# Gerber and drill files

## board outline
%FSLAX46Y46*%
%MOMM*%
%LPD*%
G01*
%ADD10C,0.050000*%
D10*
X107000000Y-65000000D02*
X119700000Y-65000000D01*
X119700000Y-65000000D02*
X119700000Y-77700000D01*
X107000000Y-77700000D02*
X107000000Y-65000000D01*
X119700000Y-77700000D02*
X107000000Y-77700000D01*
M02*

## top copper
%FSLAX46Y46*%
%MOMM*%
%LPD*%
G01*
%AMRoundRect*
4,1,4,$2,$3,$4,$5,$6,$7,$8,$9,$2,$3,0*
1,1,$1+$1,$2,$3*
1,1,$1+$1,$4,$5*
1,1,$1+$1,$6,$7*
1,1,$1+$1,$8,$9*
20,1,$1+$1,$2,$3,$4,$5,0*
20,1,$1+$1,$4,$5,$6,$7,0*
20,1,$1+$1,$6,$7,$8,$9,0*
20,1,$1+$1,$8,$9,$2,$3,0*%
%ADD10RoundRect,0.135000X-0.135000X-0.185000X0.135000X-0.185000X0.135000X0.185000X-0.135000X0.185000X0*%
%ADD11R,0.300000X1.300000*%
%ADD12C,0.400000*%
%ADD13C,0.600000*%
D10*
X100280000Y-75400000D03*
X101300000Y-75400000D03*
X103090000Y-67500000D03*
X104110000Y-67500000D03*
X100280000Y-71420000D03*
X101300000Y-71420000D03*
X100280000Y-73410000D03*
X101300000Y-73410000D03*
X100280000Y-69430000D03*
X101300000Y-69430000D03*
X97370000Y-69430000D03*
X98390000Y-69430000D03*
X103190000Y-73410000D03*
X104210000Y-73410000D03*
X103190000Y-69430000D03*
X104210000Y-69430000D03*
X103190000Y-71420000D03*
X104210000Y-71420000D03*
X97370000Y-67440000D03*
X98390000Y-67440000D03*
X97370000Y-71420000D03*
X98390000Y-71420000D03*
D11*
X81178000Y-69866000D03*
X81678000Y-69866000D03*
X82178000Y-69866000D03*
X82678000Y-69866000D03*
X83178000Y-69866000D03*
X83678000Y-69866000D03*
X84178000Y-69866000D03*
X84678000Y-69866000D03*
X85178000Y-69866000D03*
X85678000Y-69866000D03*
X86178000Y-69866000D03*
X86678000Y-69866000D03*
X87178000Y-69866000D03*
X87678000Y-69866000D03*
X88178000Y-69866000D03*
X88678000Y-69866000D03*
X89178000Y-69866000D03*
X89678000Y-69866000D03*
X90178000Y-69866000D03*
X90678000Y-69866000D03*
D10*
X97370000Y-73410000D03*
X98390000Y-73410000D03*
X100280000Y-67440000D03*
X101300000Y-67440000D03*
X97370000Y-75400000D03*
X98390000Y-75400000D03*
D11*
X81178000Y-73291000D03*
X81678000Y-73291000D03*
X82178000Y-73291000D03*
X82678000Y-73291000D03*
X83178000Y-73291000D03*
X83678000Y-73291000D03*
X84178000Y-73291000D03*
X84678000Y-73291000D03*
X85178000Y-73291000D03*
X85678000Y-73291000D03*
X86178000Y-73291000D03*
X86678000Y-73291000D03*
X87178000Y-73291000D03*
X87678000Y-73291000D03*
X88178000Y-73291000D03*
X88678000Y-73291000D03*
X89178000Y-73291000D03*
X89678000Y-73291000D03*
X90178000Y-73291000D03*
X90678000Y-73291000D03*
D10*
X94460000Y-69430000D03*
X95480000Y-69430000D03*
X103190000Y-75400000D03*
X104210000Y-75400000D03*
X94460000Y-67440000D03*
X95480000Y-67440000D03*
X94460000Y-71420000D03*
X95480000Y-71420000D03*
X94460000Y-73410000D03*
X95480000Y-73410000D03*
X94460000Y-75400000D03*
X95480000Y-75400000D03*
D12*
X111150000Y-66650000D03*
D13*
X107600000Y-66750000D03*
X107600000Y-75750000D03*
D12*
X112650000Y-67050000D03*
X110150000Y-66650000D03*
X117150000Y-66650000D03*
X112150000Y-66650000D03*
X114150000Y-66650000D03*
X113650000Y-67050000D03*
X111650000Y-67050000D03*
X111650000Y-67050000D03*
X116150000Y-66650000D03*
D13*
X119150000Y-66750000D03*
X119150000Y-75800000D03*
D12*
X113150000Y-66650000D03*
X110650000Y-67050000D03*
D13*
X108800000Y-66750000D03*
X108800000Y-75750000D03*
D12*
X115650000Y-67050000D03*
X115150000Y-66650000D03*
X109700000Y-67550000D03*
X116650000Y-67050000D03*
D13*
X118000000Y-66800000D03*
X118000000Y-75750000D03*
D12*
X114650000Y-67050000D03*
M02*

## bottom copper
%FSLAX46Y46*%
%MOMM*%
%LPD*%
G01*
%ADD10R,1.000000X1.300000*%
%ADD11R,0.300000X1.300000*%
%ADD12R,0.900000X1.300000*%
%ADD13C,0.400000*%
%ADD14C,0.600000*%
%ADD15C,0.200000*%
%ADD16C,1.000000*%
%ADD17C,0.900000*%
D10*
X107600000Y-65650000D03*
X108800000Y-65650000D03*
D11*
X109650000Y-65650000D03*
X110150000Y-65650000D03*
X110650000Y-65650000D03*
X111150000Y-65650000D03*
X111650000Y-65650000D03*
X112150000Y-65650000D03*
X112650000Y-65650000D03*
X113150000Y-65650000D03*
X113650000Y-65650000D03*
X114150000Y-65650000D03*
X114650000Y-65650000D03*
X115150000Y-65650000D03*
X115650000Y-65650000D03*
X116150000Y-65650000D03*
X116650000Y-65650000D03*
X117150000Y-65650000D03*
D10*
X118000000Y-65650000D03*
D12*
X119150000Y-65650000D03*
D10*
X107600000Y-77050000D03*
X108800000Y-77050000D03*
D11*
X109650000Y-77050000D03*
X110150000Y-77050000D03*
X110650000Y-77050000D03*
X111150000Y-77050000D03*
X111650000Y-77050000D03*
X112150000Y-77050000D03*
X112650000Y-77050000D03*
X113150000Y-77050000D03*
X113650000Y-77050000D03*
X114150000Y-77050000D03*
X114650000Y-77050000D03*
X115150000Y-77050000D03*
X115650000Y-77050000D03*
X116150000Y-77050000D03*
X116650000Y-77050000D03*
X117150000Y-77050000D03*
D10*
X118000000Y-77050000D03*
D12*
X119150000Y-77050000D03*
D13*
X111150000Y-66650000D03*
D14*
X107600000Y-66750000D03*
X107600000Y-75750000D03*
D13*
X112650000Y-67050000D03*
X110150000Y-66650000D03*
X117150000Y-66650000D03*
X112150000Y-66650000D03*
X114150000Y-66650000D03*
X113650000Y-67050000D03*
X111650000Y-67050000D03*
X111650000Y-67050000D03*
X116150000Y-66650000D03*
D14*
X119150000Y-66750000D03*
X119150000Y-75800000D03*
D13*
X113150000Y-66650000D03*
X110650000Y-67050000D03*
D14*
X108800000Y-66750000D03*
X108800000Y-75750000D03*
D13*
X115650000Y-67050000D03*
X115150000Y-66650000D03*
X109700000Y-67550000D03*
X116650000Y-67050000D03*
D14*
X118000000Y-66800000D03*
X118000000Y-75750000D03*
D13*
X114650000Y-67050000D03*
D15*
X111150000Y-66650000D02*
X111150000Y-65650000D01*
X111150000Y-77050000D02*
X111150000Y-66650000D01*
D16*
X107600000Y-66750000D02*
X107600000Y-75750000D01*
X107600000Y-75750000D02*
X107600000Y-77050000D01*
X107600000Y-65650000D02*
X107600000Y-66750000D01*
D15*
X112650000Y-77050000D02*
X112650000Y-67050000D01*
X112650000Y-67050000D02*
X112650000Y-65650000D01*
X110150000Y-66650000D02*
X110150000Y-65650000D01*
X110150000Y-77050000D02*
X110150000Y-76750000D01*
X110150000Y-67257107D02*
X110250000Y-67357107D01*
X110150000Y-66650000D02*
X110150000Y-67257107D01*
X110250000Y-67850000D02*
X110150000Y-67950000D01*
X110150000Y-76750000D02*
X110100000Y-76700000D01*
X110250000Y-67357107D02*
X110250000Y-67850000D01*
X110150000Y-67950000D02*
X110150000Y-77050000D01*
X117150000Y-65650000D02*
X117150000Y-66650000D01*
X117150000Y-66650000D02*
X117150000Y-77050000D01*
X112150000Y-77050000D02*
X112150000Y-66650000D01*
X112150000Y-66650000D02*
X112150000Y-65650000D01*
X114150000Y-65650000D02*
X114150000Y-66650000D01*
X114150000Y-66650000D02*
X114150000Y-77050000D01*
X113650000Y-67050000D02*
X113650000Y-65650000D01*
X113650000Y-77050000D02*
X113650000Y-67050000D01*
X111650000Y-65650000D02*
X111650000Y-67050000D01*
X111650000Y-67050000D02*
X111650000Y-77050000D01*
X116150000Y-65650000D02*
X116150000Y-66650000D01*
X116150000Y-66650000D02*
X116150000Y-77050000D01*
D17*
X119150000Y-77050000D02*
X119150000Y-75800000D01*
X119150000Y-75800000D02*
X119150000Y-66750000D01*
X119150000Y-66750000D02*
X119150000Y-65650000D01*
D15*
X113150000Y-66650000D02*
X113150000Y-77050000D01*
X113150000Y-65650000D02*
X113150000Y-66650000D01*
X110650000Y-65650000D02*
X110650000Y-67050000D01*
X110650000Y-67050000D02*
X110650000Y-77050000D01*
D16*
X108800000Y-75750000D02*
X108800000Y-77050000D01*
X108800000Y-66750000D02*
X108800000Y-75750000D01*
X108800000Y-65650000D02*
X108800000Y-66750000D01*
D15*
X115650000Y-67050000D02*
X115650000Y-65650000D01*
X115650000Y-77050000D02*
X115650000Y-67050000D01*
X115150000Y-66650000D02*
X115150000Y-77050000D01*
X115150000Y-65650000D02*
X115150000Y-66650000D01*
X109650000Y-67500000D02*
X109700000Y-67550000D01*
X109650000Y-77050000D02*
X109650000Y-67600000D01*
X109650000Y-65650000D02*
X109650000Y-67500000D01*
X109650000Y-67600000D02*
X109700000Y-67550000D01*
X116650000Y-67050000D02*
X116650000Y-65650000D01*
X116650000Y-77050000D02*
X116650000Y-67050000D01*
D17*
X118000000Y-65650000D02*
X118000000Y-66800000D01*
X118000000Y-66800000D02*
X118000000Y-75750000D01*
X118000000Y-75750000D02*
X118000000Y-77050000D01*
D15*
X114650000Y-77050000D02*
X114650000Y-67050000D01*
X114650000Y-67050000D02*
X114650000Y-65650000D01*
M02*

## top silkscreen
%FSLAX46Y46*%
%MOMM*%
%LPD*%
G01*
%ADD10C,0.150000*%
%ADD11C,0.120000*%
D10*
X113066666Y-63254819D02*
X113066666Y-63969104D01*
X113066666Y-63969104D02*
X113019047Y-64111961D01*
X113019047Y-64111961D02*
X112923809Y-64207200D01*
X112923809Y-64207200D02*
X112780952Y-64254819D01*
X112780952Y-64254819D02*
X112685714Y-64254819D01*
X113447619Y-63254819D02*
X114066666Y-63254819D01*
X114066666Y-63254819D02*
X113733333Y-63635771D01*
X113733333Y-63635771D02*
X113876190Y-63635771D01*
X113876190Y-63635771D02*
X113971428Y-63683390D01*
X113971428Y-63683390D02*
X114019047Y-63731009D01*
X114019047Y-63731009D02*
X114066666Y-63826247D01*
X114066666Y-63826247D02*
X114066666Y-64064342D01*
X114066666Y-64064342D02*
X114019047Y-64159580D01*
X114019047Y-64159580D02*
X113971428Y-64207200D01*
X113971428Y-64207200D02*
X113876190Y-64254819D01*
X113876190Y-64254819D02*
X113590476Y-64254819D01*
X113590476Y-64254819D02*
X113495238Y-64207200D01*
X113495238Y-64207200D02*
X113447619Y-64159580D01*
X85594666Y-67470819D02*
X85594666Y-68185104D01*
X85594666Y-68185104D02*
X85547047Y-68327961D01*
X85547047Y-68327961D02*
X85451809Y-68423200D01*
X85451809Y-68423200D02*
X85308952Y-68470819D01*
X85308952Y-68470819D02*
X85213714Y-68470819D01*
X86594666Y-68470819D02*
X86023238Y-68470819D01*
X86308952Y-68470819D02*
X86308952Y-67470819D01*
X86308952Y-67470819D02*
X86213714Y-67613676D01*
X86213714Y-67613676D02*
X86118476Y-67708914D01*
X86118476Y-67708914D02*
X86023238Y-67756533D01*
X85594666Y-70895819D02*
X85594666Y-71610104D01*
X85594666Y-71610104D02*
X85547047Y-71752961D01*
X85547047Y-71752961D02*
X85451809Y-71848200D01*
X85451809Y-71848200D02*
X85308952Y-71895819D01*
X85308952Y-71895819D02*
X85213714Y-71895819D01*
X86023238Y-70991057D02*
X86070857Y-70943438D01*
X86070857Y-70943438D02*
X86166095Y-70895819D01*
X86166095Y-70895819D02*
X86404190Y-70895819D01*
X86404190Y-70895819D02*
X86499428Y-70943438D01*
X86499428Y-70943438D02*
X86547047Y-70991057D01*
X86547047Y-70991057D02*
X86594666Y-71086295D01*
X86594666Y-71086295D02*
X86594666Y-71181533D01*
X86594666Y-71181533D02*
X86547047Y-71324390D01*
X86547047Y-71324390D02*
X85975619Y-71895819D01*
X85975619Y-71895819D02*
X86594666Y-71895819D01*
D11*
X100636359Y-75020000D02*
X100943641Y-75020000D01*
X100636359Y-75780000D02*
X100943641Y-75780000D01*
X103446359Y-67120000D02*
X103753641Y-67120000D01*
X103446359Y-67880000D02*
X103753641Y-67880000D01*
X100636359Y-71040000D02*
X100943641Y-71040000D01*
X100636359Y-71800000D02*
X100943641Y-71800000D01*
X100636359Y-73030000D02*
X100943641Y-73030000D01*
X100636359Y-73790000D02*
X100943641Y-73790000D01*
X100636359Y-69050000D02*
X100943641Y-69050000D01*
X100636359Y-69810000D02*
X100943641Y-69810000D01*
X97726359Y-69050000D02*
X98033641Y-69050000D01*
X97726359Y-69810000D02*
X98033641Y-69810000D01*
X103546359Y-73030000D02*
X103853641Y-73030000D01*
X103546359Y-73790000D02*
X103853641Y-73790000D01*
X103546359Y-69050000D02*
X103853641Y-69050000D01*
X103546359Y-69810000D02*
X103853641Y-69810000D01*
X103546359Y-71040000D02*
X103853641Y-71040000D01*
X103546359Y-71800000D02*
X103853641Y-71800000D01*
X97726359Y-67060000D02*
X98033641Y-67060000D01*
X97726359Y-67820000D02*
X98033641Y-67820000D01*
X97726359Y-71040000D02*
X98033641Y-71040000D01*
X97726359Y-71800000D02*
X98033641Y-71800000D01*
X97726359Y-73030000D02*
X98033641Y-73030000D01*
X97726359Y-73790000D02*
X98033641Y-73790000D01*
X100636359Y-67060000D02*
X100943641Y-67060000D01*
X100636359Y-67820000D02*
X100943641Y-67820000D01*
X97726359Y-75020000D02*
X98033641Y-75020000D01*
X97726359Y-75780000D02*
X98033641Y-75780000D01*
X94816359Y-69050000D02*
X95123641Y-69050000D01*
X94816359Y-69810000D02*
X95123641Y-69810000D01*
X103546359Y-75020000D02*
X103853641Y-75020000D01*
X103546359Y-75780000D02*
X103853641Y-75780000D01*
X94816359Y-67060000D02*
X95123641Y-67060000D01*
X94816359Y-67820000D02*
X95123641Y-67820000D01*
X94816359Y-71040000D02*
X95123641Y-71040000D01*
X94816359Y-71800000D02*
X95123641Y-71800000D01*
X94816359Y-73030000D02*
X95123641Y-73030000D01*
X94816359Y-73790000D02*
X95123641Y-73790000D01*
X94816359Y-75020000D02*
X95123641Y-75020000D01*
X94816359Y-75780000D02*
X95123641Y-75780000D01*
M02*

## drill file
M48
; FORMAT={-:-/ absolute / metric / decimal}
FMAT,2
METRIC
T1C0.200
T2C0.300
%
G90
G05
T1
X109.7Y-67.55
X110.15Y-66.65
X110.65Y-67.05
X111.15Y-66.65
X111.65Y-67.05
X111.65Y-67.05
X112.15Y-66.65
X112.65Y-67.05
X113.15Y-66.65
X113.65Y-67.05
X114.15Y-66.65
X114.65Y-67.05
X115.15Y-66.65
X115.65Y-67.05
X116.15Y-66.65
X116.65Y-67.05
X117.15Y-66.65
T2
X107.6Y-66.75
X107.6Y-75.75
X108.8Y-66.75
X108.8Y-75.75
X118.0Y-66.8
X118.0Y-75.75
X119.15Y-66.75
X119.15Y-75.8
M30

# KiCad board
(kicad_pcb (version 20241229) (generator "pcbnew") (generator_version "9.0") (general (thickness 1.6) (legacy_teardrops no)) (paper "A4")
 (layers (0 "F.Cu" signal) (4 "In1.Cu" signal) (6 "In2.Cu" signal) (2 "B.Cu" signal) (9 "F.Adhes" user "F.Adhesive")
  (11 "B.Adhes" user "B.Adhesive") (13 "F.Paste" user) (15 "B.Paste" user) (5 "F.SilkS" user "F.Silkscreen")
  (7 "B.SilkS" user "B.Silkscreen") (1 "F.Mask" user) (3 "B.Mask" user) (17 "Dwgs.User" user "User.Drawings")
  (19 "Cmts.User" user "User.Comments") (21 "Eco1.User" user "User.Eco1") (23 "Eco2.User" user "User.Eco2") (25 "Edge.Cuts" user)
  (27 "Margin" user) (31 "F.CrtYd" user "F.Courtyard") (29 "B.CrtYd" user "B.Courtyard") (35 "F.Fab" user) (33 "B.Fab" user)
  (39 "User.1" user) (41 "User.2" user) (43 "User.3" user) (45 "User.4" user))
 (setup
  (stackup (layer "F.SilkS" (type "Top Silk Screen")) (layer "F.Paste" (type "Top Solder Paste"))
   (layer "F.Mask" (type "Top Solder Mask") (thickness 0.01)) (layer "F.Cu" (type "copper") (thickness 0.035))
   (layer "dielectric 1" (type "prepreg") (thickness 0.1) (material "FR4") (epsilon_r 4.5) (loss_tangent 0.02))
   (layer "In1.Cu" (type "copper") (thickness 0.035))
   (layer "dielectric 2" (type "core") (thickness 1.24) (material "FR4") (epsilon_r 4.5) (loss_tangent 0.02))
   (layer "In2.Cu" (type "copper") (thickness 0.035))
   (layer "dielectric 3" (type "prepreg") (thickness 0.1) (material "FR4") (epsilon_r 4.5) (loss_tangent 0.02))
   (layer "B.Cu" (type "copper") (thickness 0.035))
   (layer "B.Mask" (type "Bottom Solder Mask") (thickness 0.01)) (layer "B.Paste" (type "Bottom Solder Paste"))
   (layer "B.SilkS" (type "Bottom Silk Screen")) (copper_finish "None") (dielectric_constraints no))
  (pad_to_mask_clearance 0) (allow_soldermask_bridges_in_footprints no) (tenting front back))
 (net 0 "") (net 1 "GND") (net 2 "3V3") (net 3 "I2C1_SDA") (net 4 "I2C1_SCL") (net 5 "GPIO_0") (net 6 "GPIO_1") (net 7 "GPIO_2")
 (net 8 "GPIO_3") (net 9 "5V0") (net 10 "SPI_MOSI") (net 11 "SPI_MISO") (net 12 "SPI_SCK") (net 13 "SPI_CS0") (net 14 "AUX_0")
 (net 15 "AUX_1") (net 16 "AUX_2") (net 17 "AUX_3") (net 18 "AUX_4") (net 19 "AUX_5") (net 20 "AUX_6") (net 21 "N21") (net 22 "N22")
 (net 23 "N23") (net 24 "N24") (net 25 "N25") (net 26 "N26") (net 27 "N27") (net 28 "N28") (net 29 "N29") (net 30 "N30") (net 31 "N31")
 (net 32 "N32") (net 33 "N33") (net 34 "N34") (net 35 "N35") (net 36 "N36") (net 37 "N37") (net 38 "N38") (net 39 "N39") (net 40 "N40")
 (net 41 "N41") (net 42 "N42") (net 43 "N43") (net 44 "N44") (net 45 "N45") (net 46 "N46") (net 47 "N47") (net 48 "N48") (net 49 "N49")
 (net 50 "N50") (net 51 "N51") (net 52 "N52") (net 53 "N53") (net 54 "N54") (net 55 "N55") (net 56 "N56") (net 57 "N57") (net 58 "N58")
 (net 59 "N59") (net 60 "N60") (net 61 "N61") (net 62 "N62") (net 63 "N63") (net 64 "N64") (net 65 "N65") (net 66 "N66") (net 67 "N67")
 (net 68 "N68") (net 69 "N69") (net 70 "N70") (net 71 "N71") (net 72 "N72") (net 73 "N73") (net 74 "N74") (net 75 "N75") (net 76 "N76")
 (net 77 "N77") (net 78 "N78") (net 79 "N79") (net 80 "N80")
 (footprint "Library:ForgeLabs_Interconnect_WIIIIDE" (layer "F.Cu") (at 113.4 66.65)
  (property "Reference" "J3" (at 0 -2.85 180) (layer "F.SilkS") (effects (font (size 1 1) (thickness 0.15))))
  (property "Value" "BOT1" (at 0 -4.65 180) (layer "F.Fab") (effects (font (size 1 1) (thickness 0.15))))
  (pad "1" smd rect (at -5.8 -1) (size 1 1.3) (layers "B.Cu" "B.Mask" "B.Paste") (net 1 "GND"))
  (pad "2" smd rect (at -4.6 -1) (size 1 1.3) (layers "B.Cu" "B.Mask" "B.Paste") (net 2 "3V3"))
  (pad "3" smd rect (at -3.75 -1) (size 0.3 1.3) (layers "B.Cu" "B.Mask" "B.Paste") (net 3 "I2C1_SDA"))
  (pad "4" smd rect (at -3.25 -1) (size 0.3 1.3) (layers "B.Cu" "B.Mask" "B.Paste") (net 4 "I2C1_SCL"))
  (pad "5" smd rect (at -2.75 -1) (size 0.3 1.3) (layers "B.Cu" "B.Mask" "B.Paste") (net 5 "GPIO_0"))
  (pad "6" smd rect (at -2.25 -1) (size 0.3 1.3) (layers "B.Cu" "B.Mask" "B.Paste") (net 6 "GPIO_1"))
  (pad "7" smd rect (at -1.75 -1) (size 0.3 1.3) (layers "B.Cu" "B.Mask" "B.Paste") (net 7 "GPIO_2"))
  (pad "8" smd rect (at -1.25 -1) (size 0.3 1.3) (layers "B.Cu" "B.Mask" "B.Paste") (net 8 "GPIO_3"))
  (pad "9" smd rect (at -0.75 -1) (size 0.3 1.3) (layers "B.Cu" "B.Mask" "B.Paste") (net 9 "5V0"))
  (pad "10" smd rect (at -0.25 -1) (size 0.3 1.3) (layers "B.Cu" "B.Mask" "B.Paste") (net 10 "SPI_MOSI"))
  (pad "11" smd rect (at 0.25 -1) (size 0.3 1.3) (layers "B.Cu" "B.Mask" "B.Paste") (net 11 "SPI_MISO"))
  (pad "12" smd rect (at 0.75 -1) (size 0.3 1.3) (layers "B.Cu" "B.Mask" "B.Paste") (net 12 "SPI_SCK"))
  (pad "13" smd rect (at 1.25 -1) (size 0.3 1.3) (layers "B.Cu" "B.Mask" "B.Paste") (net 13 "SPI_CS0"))
  (pad "14" smd rect (at 1.75 -1) (size 0.3 1.3) (layers "B.Cu" "B.Mask" "B.Paste") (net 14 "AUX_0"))
  (pad "15" smd rect (at 2.25 -1) (size 0.3 1.3) (layers "B.Cu" "B.Mask" "B.Paste") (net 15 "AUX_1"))
  (pad "16" smd rect (at 2.75 -1) (size 0.3 1.3) (layers "B.Cu" "B.Mask" "B.Paste") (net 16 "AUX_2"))
  (pad "17" smd rect (at 3.25 -1) (size 0.3 1.3) (layers "B.Cu" "B.Mask" "B.Paste") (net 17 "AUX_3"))
  (pad "18" smd rect (at 3.75 -1) (size 0.3 1.3) (layers "B.Cu" "B.Mask" "B.Paste") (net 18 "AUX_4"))
  (pad "19" smd rect (at 4.6 -1) (size 1 1.3) (layers "B.Cu" "B.Mask" "B.Paste") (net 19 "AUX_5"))
  (pad "20" smd rect (at 5.75 -1) (size 0.9 1.3) (layers "B.Cu" "B.Mask" "B.Paste") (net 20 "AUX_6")))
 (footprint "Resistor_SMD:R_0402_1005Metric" (layer "F.Cu") (at 100.79 75.4)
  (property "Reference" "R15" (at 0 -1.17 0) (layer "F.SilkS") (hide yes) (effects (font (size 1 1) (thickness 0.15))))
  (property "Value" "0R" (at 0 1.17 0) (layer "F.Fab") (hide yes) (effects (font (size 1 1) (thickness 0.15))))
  (fp_line (start -0.153641 -0.38) (end 0.153641 -0.38) (stroke (width 0.12) (type solid)) (layer "F.SilkS"))
  (fp_line (start -0.153641 0.38) (end 0.153641 0.38) (stroke (width 0.12) (type solid)) (layer "F.SilkS"))
  (pad "1" smd roundrect (at -0.51 0) (size 0.54 0.64) (layers "F.Cu" "F.Mask" "F.Paste") (roundrect_rratio 0.25) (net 15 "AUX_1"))
  (pad "2" smd roundrect (at 0.51 0) (size 0.54 0.64) (layers "F.Cu" "F.Mask" "F.Paste") (roundrect_rratio 0.25) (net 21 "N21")))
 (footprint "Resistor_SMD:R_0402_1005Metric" (layer "F.Cu") (at 103.6 67.5)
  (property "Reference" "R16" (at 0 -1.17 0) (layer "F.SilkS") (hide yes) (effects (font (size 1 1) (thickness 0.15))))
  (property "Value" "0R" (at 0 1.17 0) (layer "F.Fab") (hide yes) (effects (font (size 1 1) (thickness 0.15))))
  (fp_line (start -0.153641 -0.38) (end 0.153641 -0.38) (stroke (width 0.12) (type solid)) (layer "F.SilkS"))
  (fp_line (start -0.153641 0.38) (end 0.153641 0.38) (stroke (width 0.12) (type solid)) (layer "F.SilkS"))
  (pad "1" smd roundrect (at -0.51 0) (size 0.54 0.64) (layers "F.Cu" "F.Mask" "F.Paste") (roundrect_rratio 0.25) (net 16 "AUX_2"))
  (pad "2" smd roundrect (at 0.51 0) (size 0.54 0.64) (layers "F.Cu" "F.Mask" "F.Paste") (roundrect_rratio 0.25) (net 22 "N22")))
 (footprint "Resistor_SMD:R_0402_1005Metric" (layer "F.Cu") (at 100.79 71.42)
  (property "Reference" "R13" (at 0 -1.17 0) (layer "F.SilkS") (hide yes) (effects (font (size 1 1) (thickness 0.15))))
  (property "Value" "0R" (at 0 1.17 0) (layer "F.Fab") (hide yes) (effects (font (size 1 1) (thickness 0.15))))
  (fp_line (start -0.153641 -0.38) (end 0.153641 -0.38) (stroke (width 0.12) (type solid)) (layer "F.SilkS"))
  (fp_line (start -0.153641 0.38) (end 0.153641 0.38) (stroke (width 0.12) (type solid)) (layer "F.SilkS"))
  (pad "1" smd roundrect (at -0.51 0) (size 0.54 0.64) (layers "F.Cu" "F.Mask" "F.Paste") (roundrect_rratio 0.25) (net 13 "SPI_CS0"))
  (pad "2" smd roundrect (at 0.51 0) (size 0.54 0.64) (layers "F.Cu" "F.Mask" "F.Paste") (roundrect_rratio 0.25) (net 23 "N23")))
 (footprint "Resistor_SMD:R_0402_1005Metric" (layer "F.Cu") (at 100.79 73.41)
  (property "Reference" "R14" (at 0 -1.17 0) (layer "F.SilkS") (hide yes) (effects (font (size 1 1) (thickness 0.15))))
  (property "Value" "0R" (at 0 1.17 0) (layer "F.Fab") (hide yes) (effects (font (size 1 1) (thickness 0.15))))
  (fp_line (start -0.153641 -0.38) (end 0.153641 -0.38) (stroke (width 0.12) (type solid)) (layer "F.SilkS"))
  (fp_line (start -0.153641 0.38) (end 0.153641 0.38) (stroke (width 0.12) (type solid)) (layer "F.SilkS"))
  (pad "1" smd roundrect (at -0.51 0) (size 0.54 0.64) (layers "F.Cu" "F.Mask" "F.Paste") (roundrect_rratio 0.25) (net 14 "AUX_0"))
  (pad "2" smd roundrect (at 0.51 0) (size 0.54 0.64) (layers "F.Cu" "F.Mask" "F.Paste") (roundrect_rratio 0.25) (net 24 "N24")))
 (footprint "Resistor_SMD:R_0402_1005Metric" (layer "F.Cu") (at 100.79 69.43)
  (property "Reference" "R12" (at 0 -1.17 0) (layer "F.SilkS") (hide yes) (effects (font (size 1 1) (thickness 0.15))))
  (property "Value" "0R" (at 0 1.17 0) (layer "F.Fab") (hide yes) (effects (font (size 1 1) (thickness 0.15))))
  (fp_line (start -0.153641 -0.38) (end 0.153641 -0.38) (stroke (width 0.12) (type solid)) (layer "F.SilkS"))
  (fp_line (start -0.153641 0.38) (end 0.153641 0.38) (stroke (width 0.12) (type solid)) (layer "F.SilkS"))
  (pad "1" smd roundrect (at -0.51 0) (size 0.54 0.64) (layers "F.Cu" "F.Mask" "F.Paste") (roundrect_rratio 0.25) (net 12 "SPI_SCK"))
  (pad "2" smd roundrect (at 0.51 0) (size 0.54 0.64) (layers "F.Cu" "F.Mask" "F.Paste") (roundrect_rratio 0.25) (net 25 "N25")))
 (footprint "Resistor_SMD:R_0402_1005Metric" (layer "F.Cu") (at 97.88 69.43)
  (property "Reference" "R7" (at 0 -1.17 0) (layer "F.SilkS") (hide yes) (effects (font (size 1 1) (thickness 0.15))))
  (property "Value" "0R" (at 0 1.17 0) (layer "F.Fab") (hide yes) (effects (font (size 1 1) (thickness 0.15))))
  (fp_line (start -0.153641 -0.38) (end 0.153641 -0.38) (stroke (width 0.12) (type solid)) (layer "F.SilkS"))
  (fp_line (start -0.153641 0.38) (end 0.153641 0.38) (stroke (width 0.12) (type solid)) (layer "F.SilkS"))
  (pad "1" smd roundrect (at -0.51 0) (size 0.54 0.64) (layers "F.Cu" "F.Mask" "F.Paste") (roundrect_rratio 0.25) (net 7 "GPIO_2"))
  (pad "2" smd roundrect (at 0.51 0) (size 0.54 0.64) (layers "F.Cu" "F.Mask" "F.Paste") (roundrect_rratio 0.25) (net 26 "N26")))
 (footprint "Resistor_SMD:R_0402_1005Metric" (layer "F.Cu") (at 103.7 73.41)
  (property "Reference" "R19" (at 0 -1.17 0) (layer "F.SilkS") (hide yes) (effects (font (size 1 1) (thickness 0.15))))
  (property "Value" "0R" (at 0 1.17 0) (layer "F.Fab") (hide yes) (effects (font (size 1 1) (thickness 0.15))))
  (fp_line (start -0.153641 -0.38) (end 0.153641 -0.38) (stroke (width 0.12) (type solid)) (layer "F.SilkS"))
  (fp_line (start -0.153641 0.38) (end 0.153641 0.38) (stroke (width 0.12) (type solid)) (layer "F.SilkS"))
  (pad "1" smd roundrect (at -0.51 0) (size 0.54 0.64) (layers "F.Cu" "F.Mask" "F.Paste") (roundrect_rratio 0.25) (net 19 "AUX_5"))
  (pad "2" smd roundrect (at 0.51 0) (size 0.54 0.64) (layers "F.Cu" "F.Mask" "F.Paste") (roundrect_rratio 0.25) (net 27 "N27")))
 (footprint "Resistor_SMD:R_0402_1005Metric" (layer "F.Cu") (at 103.7 69.43)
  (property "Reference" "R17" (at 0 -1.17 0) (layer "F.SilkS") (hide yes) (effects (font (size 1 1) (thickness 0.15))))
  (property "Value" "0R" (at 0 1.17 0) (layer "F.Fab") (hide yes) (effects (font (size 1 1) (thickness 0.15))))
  (fp_line (start -0.153641 -0.38) (end 0.153641 -0.38) (stroke (width 0.12) (type solid)) (layer "F.SilkS"))
  (fp_line (start -0.153641 0.38) (end 0.153641 0.38) (stroke (width 0.12) (type solid)) (layer "F.SilkS"))
  (pad "1" smd roundrect (at -0.51 0) (size 0.54 0.64) (layers "F.Cu" "F.Mask" "F.Paste") (roundrect_rratio 0.25) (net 17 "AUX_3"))
  (pad "2" smd roundrect (at 0.51 0) (size 0.54 0.64) (layers "F.Cu" "F.Mask" "F.Paste") (roundrect_rratio 0.25) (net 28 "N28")))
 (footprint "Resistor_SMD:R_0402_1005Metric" (layer "F.Cu") (at 103.7 71.42)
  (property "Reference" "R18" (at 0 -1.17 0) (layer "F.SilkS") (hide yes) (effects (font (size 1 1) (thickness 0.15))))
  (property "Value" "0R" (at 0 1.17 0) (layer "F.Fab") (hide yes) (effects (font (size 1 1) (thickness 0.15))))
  (fp_line (start -0.153641 -0.38) (end 0.153641 -0.38) (stroke (width 0.12) (type solid)) (layer "F.SilkS"))
  (fp_line (start -0.153641 0.38) (end 0.153641 0.38) (stroke (width 0.12) (type solid)) (layer "F.SilkS"))
  (pad "1" smd roundrect (at -0.51 0) (size 0.54 0.64) (layers "F.Cu" "F.Mask" "F.Paste") (roundrect_rratio 0.25) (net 18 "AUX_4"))
  (pad "2" smd roundrect (at 0.51 0) (size 0.54 0.64) (layers "F.Cu" "F.Mask" "F.Paste") (roundrect_rratio 0.25) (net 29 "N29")))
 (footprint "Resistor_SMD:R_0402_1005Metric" (layer "F.Cu") (at 97.88 67.44)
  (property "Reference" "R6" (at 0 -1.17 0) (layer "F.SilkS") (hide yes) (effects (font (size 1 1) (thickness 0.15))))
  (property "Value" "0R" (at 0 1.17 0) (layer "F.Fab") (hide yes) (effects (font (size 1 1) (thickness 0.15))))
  (fp_line (start -0.153641 -0.38) (end 0.153641 -0.38) (stroke (width 0.12) (type solid)) (layer "F.SilkS"))
  (fp_line (start -0.153641 0.38) (end 0.153641 0.38) (stroke (width 0.12) (type solid)) (layer "F.SilkS"))
  (pad "1" smd roundrect (at -0.51 0) (size 0.54 0.64) (layers "F.Cu" "F.Mask" "F.Paste") (roundrect_rratio 0.25) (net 6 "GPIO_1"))
  (pad "2" smd roundrect (at 0.51 0) (size 0.54 0.64) (layers "F.Cu" "F.Mask" "F.Paste") (roundrect_rratio 0.25) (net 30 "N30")))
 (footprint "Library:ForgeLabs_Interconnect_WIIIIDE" (layer "F.Cu") (at 113.4 78.05)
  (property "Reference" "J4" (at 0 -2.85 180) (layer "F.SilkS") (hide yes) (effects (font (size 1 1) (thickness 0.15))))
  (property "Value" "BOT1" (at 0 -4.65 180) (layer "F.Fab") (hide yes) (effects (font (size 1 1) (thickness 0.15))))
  (pad "1" smd rect (at -5.8 -1) (size 1 1.3) (layers "B.Cu" "B.Mask" "B.Paste") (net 1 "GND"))
  (pad "2" smd rect (at -4.6 -1) (size 1 1.3) (layers "B.Cu" "B.Mask" "B.Paste") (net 2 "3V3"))
  (pad "3" smd rect (at -3.75 -1) (size 0.3 1.3) (layers "B.Cu" "B.Mask" "B.Paste") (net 3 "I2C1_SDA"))
  (pad "4" smd rect (at -3.25 -1) (size 0.3 1.3) (layers "B.Cu" "B.Mask" "B.Paste") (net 4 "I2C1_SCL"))
  (pad "5" smd rect (at -2.75 -1) (size 0.3 1.3) (layers "B.Cu" "B.Mask" "B.Paste") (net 5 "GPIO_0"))
  (pad "6" smd rect (at -2.25 -1) (size 0.3 1.3) (layers "B.Cu" "B.Mask" "B.Paste") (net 6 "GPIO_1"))
  (pad "7" smd rect (at -1.75 -1) (size 0.3 1.3) (layers "B.Cu" "B.Mask" "B.Paste") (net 7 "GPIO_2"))
  (pad "8" smd rect (at -1.25 -1) (size 0.3 1.3) (layers "B.Cu" "B.Mask" "B.Paste") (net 8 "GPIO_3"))
  (pad "9" smd rect (at -0.75 -1) (size 0.3 1.3) (layers "B.Cu" "B.Mask" "B.Paste") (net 9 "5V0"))
  (pad "10" smd rect (at -0.25 -1) (size 0.3 1.3) (layers "B.Cu" "B.Mask" "B.Paste") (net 10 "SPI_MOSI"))
  (pad "11" smd rect (at 0.25 -1) (size 0.3 1.3) (layers "B.Cu" "B.Mask" "B.Paste") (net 11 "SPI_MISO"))
  (pad "12" smd rect (at 0.75 -1) (size 0.3 1.3) (layers "B.Cu" "B.Mask" "B.Paste") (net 12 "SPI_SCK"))
  (pad "13" smd rect (at 1.25 -1) (size 0.3 1.3) (layers "B.Cu" "B.Mask" "B.Paste") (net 13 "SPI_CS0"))
  (pad "14" smd rect (at 1.75 -1) (size 0.3 1.3) (layers "B.Cu" "B.Mask" "B.Paste") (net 14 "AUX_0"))
  (pad "15" smd rect (at 2.25 -1) (size 0.3 1.3) (layers "B.Cu" "B.Mask" "B.Paste") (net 15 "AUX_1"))
  (pad "16" smd rect (at 2.75 -1) (size 0.3 1.3) (layers "B.Cu" "B.Mask" "B.Paste") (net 16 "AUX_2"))
  (pad "17" smd rect (at 3.25 -1) (size 0.3 1.3) (layers "B.Cu" "B.Mask" "B.Paste") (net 17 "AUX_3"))
  (pad "18" smd rect (at 3.75 -1) (size 0.3 1.3) (layers "B.Cu" "B.Mask" "B.Paste") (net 18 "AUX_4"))
  (pad "19" smd rect (at 4.6 -1) (size 1 1.3) (layers "B.Cu" "B.Mask" "B.Paste") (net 19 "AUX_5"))
  (pad "20" smd rect (at 5.75 -1) (size 0.9 1.3) (layers "B.Cu" "B.Mask" "B.Paste") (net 20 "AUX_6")))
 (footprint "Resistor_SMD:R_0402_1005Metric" (layer "F.Cu") (at 97.88 71.42)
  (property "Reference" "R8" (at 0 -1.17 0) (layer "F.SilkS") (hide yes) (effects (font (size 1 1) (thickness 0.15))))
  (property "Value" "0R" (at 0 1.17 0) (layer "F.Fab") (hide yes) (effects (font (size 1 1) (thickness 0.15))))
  (fp_line (start -0.153641 -0.38) (end 0.153641 -0.38) (stroke (width 0.12) (type solid)) (layer "F.SilkS"))
  (fp_line (start -0.153641 0.38) (end 0.153641 0.38) (stroke (width 0.12) (type solid)) (layer "F.SilkS"))
  (pad "1" smd roundrect (at -0.51 0) (size 0.54 0.64) (layers "F.Cu" "F.Mask" "F.Paste") (roundrect_rratio 0.25) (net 8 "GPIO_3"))
  (pad "2" smd roundrect (at 0.51 0) (size 0.54 0.64) (layers "F.Cu" "F.Mask" "F.Paste") (roundrect_rratio 0.25) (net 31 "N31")))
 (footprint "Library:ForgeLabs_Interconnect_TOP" (layer "F.Cu") (at 85.928 70.866)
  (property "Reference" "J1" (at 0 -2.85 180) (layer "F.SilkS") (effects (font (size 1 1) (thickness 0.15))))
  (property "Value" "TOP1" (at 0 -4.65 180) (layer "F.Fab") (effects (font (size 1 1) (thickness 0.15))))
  (pad "1" smd rect (at -4.75 -1) (size 0.3 1.3) (layers "F.Cu" "F.Mask" "F.Paste") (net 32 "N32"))
  (pad "2" smd rect (at -4.25 -1) (size 0.3 1.3) (layers "F.Cu" "F.Mask" "F.Paste") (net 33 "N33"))
  (pad "3" smd rect (at -3.75 -1) (size 0.3 1.3) (layers "F.Cu" "F.Mask" "F.Paste") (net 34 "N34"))
  (pad "4" smd rect (at -3.25 -1) (size 0.3 1.3) (layers "F.Cu" "F.Mask" "F.Paste") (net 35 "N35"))
  (pad "5" smd rect (at -2.75 -1) (size 0.3 1.3) (layers "F.Cu" "F.Mask" "F.Paste") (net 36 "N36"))
  (pad "6" smd rect (at -2.25 -1) (size 0.3 1.3) (layers "F.Cu" "F.Mask" "F.Paste") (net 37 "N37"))
  (pad "7" smd rect (at -1.75 -1) (size 0.3 1.3) (layers "F.Cu" "F.Mask" "F.Paste") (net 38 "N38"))
  (pad "8" smd rect (at -1.25 -1) (size 0.3 1.3) (layers "F.Cu" "F.Mask" "F.Paste") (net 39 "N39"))
  (pad "9" smd rect (at -0.75 -1) (size 0.3 1.3) (layers "F.Cu" "F.Mask" "F.Paste") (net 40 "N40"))
  (pad "10" smd rect (at -0.25 -1) (size 0.3 1.3) (layers "F.Cu" "F.Mask" "F.Paste") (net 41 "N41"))
  (pad "11" smd rect (at 0.25 -1) (size 0.3 1.3) (layers "F.Cu" "F.Mask" "F.Paste") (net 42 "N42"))
  (pad "12" smd rect (at 0.75 -1) (size 0.3 1.3) (layers "F.Cu" "F.Mask" "F.Paste") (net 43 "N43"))
  (pad "13" smd rect (at 1.25 -1) (size 0.3 1.3) (layers "F.Cu" "F.Mask" "F.Paste") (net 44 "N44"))
  (pad "14" smd rect (at 1.75 -1) (size 0.3 1.3) (layers "F.Cu" "F.Mask" "F.Paste") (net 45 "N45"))
  (pad "15" smd rect (at 2.25 -1) (size 0.3 1.3) (layers "F.Cu" "F.Mask" "F.Paste") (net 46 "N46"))
  (pad "16" smd rect (at 2.75 -1) (size 0.3 1.3) (layers "F.Cu" "F.Mask" "F.Paste") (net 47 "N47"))
  (pad "17" smd rect (at 3.25 -1) (size 0.3 1.3) (layers "F.Cu" "F.Mask" "F.Paste") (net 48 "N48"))
  (pad "18" smd rect (at 3.75 -1) (size 0.3 1.3) (layers "F.Cu" "F.Mask" "F.Paste") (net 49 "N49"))
  (pad "19" smd rect (at 4.25 -1) (size 0.3 1.3) (layers "F.Cu" "F.Mask" "F.Paste") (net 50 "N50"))
  (pad "20" smd rect (at 4.75 -1) (size 0.3 1.3) (layers "F.Cu" "F.Mask" "F.Paste") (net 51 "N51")))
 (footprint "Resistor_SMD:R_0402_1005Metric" (layer "F.Cu") (at 97.88 73.41)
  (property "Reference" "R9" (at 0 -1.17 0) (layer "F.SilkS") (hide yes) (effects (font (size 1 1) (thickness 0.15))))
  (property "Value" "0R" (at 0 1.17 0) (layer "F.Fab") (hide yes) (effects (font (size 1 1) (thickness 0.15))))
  (fp_line (start -0.153641 -0.38) (end 0.153641 -0.38) (stroke (width 0.12) (type solid)) (layer "F.SilkS"))
  (fp_line (start -0.153641 0.38) (end 0.153641 0.38) (stroke (width 0.12) (type solid)) (layer "F.SilkS"))
  (pad "1" smd roundrect (at -0.51 0) (size 0.54 0.64) (layers "F.Cu" "F.Mask" "F.Paste") (roundrect_rratio 0.25) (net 9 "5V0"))
  (pad "2" smd roundrect (at 0.51 0) (size 0.54 0.64) (layers "F.Cu" "F.Mask" "F.Paste") (roundrect_rratio 0.25) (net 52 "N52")))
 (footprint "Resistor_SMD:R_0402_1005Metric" (layer "F.Cu") (at 100.79 67.44)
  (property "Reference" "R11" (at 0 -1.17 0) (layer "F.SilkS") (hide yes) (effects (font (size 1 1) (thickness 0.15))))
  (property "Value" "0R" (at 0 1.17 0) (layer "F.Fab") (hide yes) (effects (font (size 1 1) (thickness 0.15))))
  (fp_line (start -0.153641 -0.38) (end 0.153641 -0.38) (stroke (width 0.12) (type solid)) (layer "F.SilkS"))
  (fp_line (start -0.153641 0.38) (end 0.153641 0.38) (stroke (width 0.12) (type solid)) (layer "F.SilkS"))
  (pad "1" smd roundrect (at -0.51 0) (size 0.54 0.64) (layers "F.Cu" "F.Mask" "F.Paste") (roundrect_rratio 0.25) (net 11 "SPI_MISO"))
  (pad "2" smd roundrect (at 0.51 0) (size 0.54 0.64) (layers "F.Cu" "F.Mask" "F.Paste") (roundrect_rratio 0.25) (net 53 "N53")))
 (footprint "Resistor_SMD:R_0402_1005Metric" (layer "F.Cu") (at 97.88 75.4)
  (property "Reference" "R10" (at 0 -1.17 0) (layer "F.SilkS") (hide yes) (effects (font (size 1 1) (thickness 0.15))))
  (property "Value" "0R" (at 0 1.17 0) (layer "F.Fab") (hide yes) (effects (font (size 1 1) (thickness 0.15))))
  (fp_line (start -0.153641 -0.38) (end 0.153641 -0.38) (stroke (width 0.12) (type solid)) (layer "F.SilkS"))
  (fp_line (start -0.153641 0.38) (end 0.153641 0.38) (stroke (width 0.12) (type solid)) (layer "F.SilkS"))
  (pad "1" smd roundrect (at -0.51 0) (size 0.54 0.64) (layers "F.Cu" "F.Mask" "F.Paste") (roundrect_rratio 0.25) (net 10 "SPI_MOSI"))
  (pad "2" smd roundrect (at 0.51 0) (size 0.54 0.64) (layers "F.Cu" "F.Mask" "F.Paste") (roundrect_rratio 0.25) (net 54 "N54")))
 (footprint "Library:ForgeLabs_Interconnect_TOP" (layer "F.Cu") (at 85.928 74.291)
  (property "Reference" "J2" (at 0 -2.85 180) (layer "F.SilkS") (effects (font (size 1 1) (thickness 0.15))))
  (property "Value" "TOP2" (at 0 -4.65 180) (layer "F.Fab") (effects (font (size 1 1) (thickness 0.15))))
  (pad "1" smd rect (at -4.75 -1) (size 0.3 1.3) (layers "F.Cu" "F.Mask" "F.Paste") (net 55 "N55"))
  (pad "2" smd rect (at -4.25 -1) (size 0.3 1.3) (layers "F.Cu" "F.Mask" "F.Paste") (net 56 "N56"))
  (pad "3" smd rect (at -3.75 -1) (size 0.3 1.3) (layers "F.Cu" "F.Mask" "F.Paste") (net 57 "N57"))
  (pad "4" smd rect (at -3.25 -1) (size 0.3 1.3) (layers "F.Cu" "F.Mask" "F.Paste") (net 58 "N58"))
  (pad "5" smd rect (at -2.75 -1) (size 0.3 1.3) (layers "F.Cu" "F.Mask" "F.Paste") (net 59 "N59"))
  (pad "6" smd rect (at -2.25 -1) (size 0.3 1.3) (layers "F.Cu" "F.Mask" "F.Paste") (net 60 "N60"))
  (pad "7" smd rect (at -1.75 -1) (size 0.3 1.3) (layers "F.Cu" "F.Mask" "F.Paste") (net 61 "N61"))
  (pad "8" smd rect (at -1.25 -1) (size 0.3 1.3) (layers "F.Cu" "F.Mask" "F.Paste") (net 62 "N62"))
  (pad "9" smd rect (at -0.75 -1) (size 0.3 1.3) (layers "F.Cu" "F.Mask" "F.Paste") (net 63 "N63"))
  (pad "10" smd rect (at -0.25 -1) (size 0.3 1.3) (layers "F.Cu" "F.Mask" "F.Paste") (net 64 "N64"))
  (pad "11" smd rect (at 0.25 -1) (size 0.3 1.3) (layers "F.Cu" "F.Mask" "F.Paste") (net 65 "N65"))
  (pad "12" smd rect (at 0.75 -1) (size 0.3 1.3) (layers "F.Cu" "F.Mask" "F.Paste") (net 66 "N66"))
  (pad "13" smd rect (at 1.25 -1) (size 0.3 1.3) (layers "F.Cu" "F.Mask" "F.Paste") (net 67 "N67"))
  (pad "14" smd rect (at 1.75 -1) (size 0.3 1.3) (layers "F.Cu" "F.Mask" "F.Paste") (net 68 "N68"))
  (pad "15" smd rect (at 2.25 -1) (size 0.3 1.3) (layers "F.Cu" "F.Mask" "F.Paste") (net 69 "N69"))
  (pad "16" smd rect (at 2.75 -1) (size 0.3 1.3) (layers "F.Cu" "F.Mask" "F.Paste") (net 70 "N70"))
  (pad "17" smd rect (at 3.25 -1) (size 0.3 1.3) (layers "F.Cu" "F.Mask" "F.Paste") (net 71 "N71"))
  (pad "18" smd rect (at 3.75 -1) (size 0.3 1.3) (layers "F.Cu" "F.Mask" "F.Paste") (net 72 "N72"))
  (pad "19" smd rect (at 4.25 -1) (size 0.3 1.3) (layers "F.Cu" "F.Mask" "F.Paste") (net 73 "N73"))
  (pad "20" smd rect (at 4.75 -1) (size 0.3 1.3) (layers "F.Cu" "F.Mask" "F.Paste") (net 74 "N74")))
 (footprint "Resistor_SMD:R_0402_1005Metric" (layer "F.Cu") (at 94.97 69.43)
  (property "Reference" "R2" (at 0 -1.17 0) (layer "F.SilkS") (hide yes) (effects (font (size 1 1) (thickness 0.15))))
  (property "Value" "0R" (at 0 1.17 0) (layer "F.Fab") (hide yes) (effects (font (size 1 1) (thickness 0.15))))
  (fp_line (start -0.153641 -0.38) (end 0.153641 -0.38) (stroke (width 0.12) (type solid)) (layer "F.SilkS"))
  (fp_line (start -0.153641 0.38) (end 0.153641 0.38) (stroke (width 0.12) (type solid)) (layer "F.SilkS"))
  (pad "1" smd roundrect (at -0.51 0) (size 0.54 0.64) (layers "F.Cu" "F.Mask" "F.Paste") (roundrect_rratio 0.25) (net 2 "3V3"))
  (pad "2" smd roundrect (at 0.51 0) (size 0.54 0.64) (layers "F.Cu" "F.Mask" "F.Paste") (roundrect_rratio 0.25) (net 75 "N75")))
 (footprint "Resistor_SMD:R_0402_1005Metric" (layer "F.Cu") (at 103.7 75.4)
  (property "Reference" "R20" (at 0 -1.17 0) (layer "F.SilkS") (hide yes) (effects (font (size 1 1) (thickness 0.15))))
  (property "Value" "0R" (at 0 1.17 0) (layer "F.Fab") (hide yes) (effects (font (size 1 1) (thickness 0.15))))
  (fp_line (start -0.153641 -0.38) (end 0.153641 -0.38) (stroke (width 0.12) (type solid)) (layer "F.SilkS"))
  (fp_line (start -0.153641 0.38) (end 0.153641 0.38) (stroke (width 0.12) (type solid)) (layer "F.SilkS"))
  (pad "1" smd roundrect (at -0.51 0) (size 0.54 0.64) (layers "F.Cu" "F.Mask" "F.Paste") (roundrect_rratio 0.25) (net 20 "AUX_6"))
  (pad "2" smd roundrect (at 0.51 0) (size 0.54 0.64) (layers "F.Cu" "F.Mask" "F.Paste") (roundrect_rratio 0.25) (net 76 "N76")))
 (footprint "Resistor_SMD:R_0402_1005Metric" (layer "F.Cu") (at 94.97 67.44)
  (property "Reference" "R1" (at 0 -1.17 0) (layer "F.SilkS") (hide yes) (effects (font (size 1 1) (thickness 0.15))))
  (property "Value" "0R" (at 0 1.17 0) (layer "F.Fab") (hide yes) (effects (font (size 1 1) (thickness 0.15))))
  (fp_line (start -0.153641 -0.38) (end 0.153641 -0.38) (stroke (width 0.12) (type solid)) (layer "F.SilkS"))
  (fp_line (start -0.153641 0.38) (end 0.153641 0.38) (stroke (width 0.12) (type solid)) (layer "F.SilkS"))
  (pad "1" smd roundrect (at -0.51 0) (size 0.54 0.64) (layers "F.Cu" "F.Mask" "F.Paste") (roundrect_rratio 0.25) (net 1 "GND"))
  (pad "2" smd roundrect (at 0.51 0) (size 0.54 0.64) (layers "F.Cu" "F.Mask" "F.Paste") (roundrect_rratio 0.25) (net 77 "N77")))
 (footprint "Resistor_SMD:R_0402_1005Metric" (layer "F.Cu") (at 94.97 71.42)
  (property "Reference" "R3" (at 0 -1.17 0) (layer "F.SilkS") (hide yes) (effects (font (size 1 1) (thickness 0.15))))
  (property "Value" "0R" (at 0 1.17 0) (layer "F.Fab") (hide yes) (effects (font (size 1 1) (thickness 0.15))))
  (fp_line (start -0.153641 -0.38) (end 0.153641 -0.38) (stroke (width 0.12) (type solid)) (layer "F.SilkS"))
  (fp_line (start -0.153641 0.38) (end 0.153641 0.38) (stroke (width 0.12) (type solid)) (layer "F.SilkS"))
  (pad "1" smd roundrect (at -0.51 0) (size 0.54 0.64) (layers "F.Cu" "F.Mask" "F.Paste") (roundrect_rratio 0.25) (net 3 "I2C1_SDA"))
  (pad "2" smd roundrect (at 0.51 0) (size 0.54 0.64) (layers "F.Cu" "F.Mask" "F.Paste") (roundrect_rratio 0.25) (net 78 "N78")))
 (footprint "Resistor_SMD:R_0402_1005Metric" (layer "F.Cu") (at 94.97 73.41)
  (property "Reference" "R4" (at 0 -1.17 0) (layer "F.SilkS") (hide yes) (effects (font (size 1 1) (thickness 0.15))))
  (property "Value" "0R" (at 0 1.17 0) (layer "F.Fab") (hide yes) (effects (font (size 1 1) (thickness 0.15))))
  (fp_line (start -0.153641 -0.38) (end 0.153641 -0.38) (stroke (width 0.12) (type solid)) (layer "F.SilkS"))
  (fp_line (start -0.153641 0.38) (end 0.153641 0.38) (stroke (width 0.12) (type solid)) (layer "F.SilkS"))
  (pad "1" smd roundrect (at -0.51 0) (size 0.54 0.64) (layers "F.Cu" "F.Mask" "F.Paste") (roundrect_rratio 0.25) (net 4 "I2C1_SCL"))
  (pad "2" smd roundrect (at 0.51 0) (size 0.54 0.64) (layers "F.Cu" "F.Mask" "F.Paste") (roundrect_rratio 0.25) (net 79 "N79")))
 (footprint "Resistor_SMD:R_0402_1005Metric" (layer "F.Cu") (at 94.97 75.4)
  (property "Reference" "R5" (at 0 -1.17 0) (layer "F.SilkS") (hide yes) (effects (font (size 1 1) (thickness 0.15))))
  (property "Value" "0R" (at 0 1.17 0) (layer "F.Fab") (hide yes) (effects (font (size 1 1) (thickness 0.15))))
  (fp_line (start -0.153641 -0.38) (end 0.153641 -0.38) (stroke (width 0.12) (type solid)) (layer "F.SilkS"))
  (fp_line (start -0.153641 0.38) (end 0.153641 0.38) (stroke (width 0.12) (type solid)) (layer "F.SilkS"))
  (pad "1" smd roundrect (at -0.51 0) (size 0.54 0.64) (layers "F.Cu" "F.Mask" "F.Paste") (roundrect_rratio 0.25) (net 5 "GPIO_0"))
  (pad "2" smd roundrect (at 0.51 0) (size 0.54 0.64) (layers "F.Cu" "F.Mask" "F.Paste") (roundrect_rratio 0.25) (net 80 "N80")))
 (gr_line (start 107 65) (end 119.7 65) (stroke (width 0.05) (type default)) (layer "Edge.Cuts"))
 (gr_line (start 119.7 65) (end 119.7 77.7) (stroke (width 0.05) (type default)) (layer "Edge.Cuts"))
 (gr_line (start 107 77.7) (end 107 65) (stroke (width 0.05) (type default)) (layer "Edge.Cuts"))
 (gr_line (start 119.7 77.7) (end 107 77.7) (stroke (width 0.05) (type default)) (layer "Edge.Cuts"))
 (via (at 111.15 66.65) (size 0.4) (drill 0.2) (layers "F.Cu" "B.Cu") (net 6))
 (segment (start 111.15 66.65) (end 111.15 65.65) (width 0.2) (layer "B.Cu") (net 6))
 (segment (start 111.15 77.05) (end 111.15 66.65) (width 0.2) (layer "B.Cu") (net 6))
 (via (at 107.6 66.75) (size 0.6) (drill 0.3) (layers "F.Cu" "B.Cu") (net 1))
 (via (at 107.6 75.75) (size 0.6) (drill 0.3) (layers "F.Cu" "B.Cu") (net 1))
 (segment (start 107.6 66.75) (end 107.6 75.75) (width 1) (layer "B.Cu") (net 1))
 (segment (start 107.6 75.75) (end 107.6 77.05) (width 1) (layer "B.Cu") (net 1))
 (segment (start 107.6 65.65) (end 107.6 66.75) (width 1) (layer "B.Cu") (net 1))
 (via (at 112.65 67.05) (size 0.4) (drill 0.2) (layers "F.Cu" "B.Cu") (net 9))
 (segment (start 112.65 77.05) (end 112.65 67.05) (width 0.2) (layer "B.Cu") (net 9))
 (segment (start 112.65 67.05) (end 112.65 65.65) (width 0.2) (layer "B.Cu") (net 9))
 (via (at 110.15 66.65) (size 0.4) (drill 0.2) (layers "F.Cu" "B.Cu") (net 4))
 (segment (start 110.15 66.65) (end 110.15 65.65) (width 0.2) (layer "B.Cu") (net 4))
 (segment (start 110.15 77.05) (end 110.15 76.75) (width 0.2) (layer "B.Cu") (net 4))
 (segment (start 110.15 67.257107) (end 110.25 67.357107) (width 0.2) (layer "B.Cu") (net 4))
 (segment (start 110.15 66.65) (end 110.15 67.257107) (width 0.2) (layer "B.Cu") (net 4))
 (segment (start 110.25 67.85) (end 110.15 67.95) (width 0.2) (layer "B.Cu") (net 4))
 (segment (start 110.15 76.75) (end 110.1 76.7) (width 0.2) (layer "B.Cu") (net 4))
 (segment (start 110.25 67.357107) (end 110.25 67.85) (width 0.2) (layer "B.Cu") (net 4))
 (segment (start 110.15 67.95) (end 110.15 77.05) (width 0.2) (layer "B.Cu") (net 4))
 (via (at 117.15 66.65) (size 0.4) (drill 0.2) (layers "F.Cu" "B.Cu") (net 18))
 (segment (start 117.15 65.65) (end 117.15 66.65) (width 0.2) (layer "B.Cu") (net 18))
 (segment (start 117.15 66.65) (end 117.15 77.05) (width 0.2) (layer "B.Cu") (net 18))
 (via (at 112.15 66.65) (size 0.4) (drill 0.2) (layers "F.Cu" "B.Cu") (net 8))
 (segment (start 112.15 77.05) (end 112.15 66.65) (width 0.2) (layer "B.Cu") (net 8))
 (segment (start 112.15 66.65) (end 112.15 65.65) (width 0.2) (layer "B.Cu") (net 8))
 (via (at 114.15 66.65) (size 0.4) (drill 0.2) (layers "F.Cu" "B.Cu") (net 12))
 (segment (start 114.15 65.65) (end 114.15 66.65) (width 0.2) (layer "B.Cu") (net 12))
 (segment (start 114.15 66.65) (end 114.15 77.05) (width 0.2) (layer "B.Cu") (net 12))
 (via (at 113.65 67.05) (size 0.4) (drill 0.2) (layers "F.Cu" "B.Cu") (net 11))
 (segment (start 113.65 67.05) (end 113.65 65.65) (width 0.2) (layer "B.Cu") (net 11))
 (segment (start 113.65 77.05) (end 113.65 67.05) (width 0.2) (layer "B.Cu") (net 11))
 (via (at 111.65 67.05) (size 0.4) (drill 0.2) (layers "F.Cu" "B.Cu") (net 7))
 (via (at 111.65 67.05) (size 0.4) (drill 0.2) (layers "F.Cu" "B.Cu") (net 7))
 (segment (start 111.65 65.65) (end 111.65 67.05) (width 0.2) (layer "B.Cu") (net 7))
 (segment (start 111.65 67.05) (end 111.65 77.05) (width 0.2) (layer "B.Cu") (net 7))
 (via (at 116.15 66.65) (size 0.4) (drill 0.2) (layers "F.Cu" "B.Cu") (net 16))
 (segment (start 116.15 65.65) (end 116.15 66.65) (width 0.2) (layer "B.Cu") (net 16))
 (segment (start 116.15 66.65) (end 116.15 77.05) (width 0.2) (layer "B.Cu") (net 16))
 (via (at 119.15 66.75) (size 0.6) (drill 0.3) (layers "F.Cu" "B.Cu") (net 20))
 (via (at 119.15 75.8) (size 0.6) (drill 0.3) (layers "F.Cu" "B.Cu") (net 20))
 (segment (start 119.15 77.05) (end 119.15 75.8) (width 0.9) (layer "B.Cu") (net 20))
 (segment (start 119.15 75.8) (end 119.15 66.75) (width 0.9) (layer "B.Cu") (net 20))
 (segment (start 119.15 66.75) (end 119.15 65.65) (width 0.9) (layer "B.Cu") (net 20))
 (via (at 113.15 66.65) (size 0.4) (drill 0.2) (layers "F.Cu" "B.Cu") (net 10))
 (segment (start 113.15 66.65) (end 113.15 77.05) (width 0.2) (layer "B.Cu") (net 10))
 (segment (start 113.15 65.65) (end 113.15 66.65) (width 0.2) (layer "B.Cu") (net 10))
 (via (at 110.65 67.05) (size 0.4) (drill 0.2) (layers "F.Cu" "B.Cu") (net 5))
 (segment (start 110.65 65.65) (end 110.65 67.05) (width 0.2) (layer "B.Cu") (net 5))
 (segment (start 110.65 67.05) (end 110.65 77.05) (width 0.2) (layer "B.Cu") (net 5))
 (via (at 108.8 66.75) (size 0.6) (drill 0.3) (layers "F.Cu" "B.Cu") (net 2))
 (via (at 108.8 75.75) (size 0.6) (drill 0.3) (layers "F.Cu" "B.Cu") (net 2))
 (segment (start 108.8 75.75) (end 108.8 77.05) (width 1) (layer "B.Cu") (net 2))
 (segment (start 108.8 66.75) (end 108.8 75.75) (width 1) (layer "B.Cu") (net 2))
 (segment (start 108.8 65.65) (end 108.8 66.75) (width 1) (layer "B.Cu") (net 2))
 (via (at 115.65 67.05) (size 0.4) (drill 0.2) (layers "F.Cu" "B.Cu") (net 15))
 (segment (start 115.65 67.05) (end 115.65 65.65) (width 0.2) (layer "B.Cu") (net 15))
 (segment (start 115.65 77.05) (end 115.65 67.05) (width 0.2) (layer "B.Cu") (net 15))
 (via (at 115.15 66.65) (size 0.4) (drill 0.2) (layers "F.Cu" "B.Cu") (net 14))
 (segment (start 115.15 66.65) (end 115.15 77.05) (width 0.2) (layer "B.Cu") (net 14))
 (segment (start 115.15 65.65) (end 115.15 66.65) (width 0.2) (layer "B.Cu") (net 14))
 (via (at 109.7 67.55) (size 0.4) (drill 0.2) (layers "F.Cu" "B.Cu") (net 3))
 (segment (start 109.65 67.5) (end 109.7 67.55) (width 0.2) (layer "B.Cu") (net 3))
 (segment (start 109.65 77.05) (end 109.65 67.6) (width 0.2) (layer "B.Cu") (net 3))
 (segment (start 109.65 65.65) (end 109.65 67.5) (width 0.2) (layer "B.Cu") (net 3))
 (segment (start 109.65 67.6) (end 109.7 67.55) (width 0.2) (layer "B.Cu") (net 3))
 (via (at 116.65 67.05) (size 0.4) (drill 0.2) (layers "F.Cu" "B.Cu") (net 17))
 (segment (start 116.65 67.05) (end 116.65 65.65) (width 0.2) (layer "B.Cu") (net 17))
 (segment (start 116.65 77.05) (end 116.65 67.05) (width 0.2) (layer "B.Cu") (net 17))
 (via (at 118 66.8) (size 0.6) (drill 0.3) (layers "F.Cu" "B.Cu") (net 19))
 (via (at 118 75.75) (size 0.6) (drill 0.3) (layers "F.Cu" "B.Cu") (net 19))
 (segment (start 118 65.65) (end 118 66.8) (width 0.9) (layer "B.Cu") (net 19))
 (segment (start 118 66.8) (end 118 75.75) (width 0.9) (layer "B.Cu") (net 19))
 (segment (start 118 75.75) (end 118 77.05) (width 0.9) (layer "B.Cu") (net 19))
 (via (at 114.65 67.05) (size 0.4) (drill 0.2) (layers "F.Cu" "B.Cu") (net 13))
 (segment (start 114.65 77.05) (end 114.65 67.05) (width 0.2) (layer "B.Cu") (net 13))
 (segment (start 114.65 67.05) (end 114.65 65.65) (width 0.2) (layer "B.Cu") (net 13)))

